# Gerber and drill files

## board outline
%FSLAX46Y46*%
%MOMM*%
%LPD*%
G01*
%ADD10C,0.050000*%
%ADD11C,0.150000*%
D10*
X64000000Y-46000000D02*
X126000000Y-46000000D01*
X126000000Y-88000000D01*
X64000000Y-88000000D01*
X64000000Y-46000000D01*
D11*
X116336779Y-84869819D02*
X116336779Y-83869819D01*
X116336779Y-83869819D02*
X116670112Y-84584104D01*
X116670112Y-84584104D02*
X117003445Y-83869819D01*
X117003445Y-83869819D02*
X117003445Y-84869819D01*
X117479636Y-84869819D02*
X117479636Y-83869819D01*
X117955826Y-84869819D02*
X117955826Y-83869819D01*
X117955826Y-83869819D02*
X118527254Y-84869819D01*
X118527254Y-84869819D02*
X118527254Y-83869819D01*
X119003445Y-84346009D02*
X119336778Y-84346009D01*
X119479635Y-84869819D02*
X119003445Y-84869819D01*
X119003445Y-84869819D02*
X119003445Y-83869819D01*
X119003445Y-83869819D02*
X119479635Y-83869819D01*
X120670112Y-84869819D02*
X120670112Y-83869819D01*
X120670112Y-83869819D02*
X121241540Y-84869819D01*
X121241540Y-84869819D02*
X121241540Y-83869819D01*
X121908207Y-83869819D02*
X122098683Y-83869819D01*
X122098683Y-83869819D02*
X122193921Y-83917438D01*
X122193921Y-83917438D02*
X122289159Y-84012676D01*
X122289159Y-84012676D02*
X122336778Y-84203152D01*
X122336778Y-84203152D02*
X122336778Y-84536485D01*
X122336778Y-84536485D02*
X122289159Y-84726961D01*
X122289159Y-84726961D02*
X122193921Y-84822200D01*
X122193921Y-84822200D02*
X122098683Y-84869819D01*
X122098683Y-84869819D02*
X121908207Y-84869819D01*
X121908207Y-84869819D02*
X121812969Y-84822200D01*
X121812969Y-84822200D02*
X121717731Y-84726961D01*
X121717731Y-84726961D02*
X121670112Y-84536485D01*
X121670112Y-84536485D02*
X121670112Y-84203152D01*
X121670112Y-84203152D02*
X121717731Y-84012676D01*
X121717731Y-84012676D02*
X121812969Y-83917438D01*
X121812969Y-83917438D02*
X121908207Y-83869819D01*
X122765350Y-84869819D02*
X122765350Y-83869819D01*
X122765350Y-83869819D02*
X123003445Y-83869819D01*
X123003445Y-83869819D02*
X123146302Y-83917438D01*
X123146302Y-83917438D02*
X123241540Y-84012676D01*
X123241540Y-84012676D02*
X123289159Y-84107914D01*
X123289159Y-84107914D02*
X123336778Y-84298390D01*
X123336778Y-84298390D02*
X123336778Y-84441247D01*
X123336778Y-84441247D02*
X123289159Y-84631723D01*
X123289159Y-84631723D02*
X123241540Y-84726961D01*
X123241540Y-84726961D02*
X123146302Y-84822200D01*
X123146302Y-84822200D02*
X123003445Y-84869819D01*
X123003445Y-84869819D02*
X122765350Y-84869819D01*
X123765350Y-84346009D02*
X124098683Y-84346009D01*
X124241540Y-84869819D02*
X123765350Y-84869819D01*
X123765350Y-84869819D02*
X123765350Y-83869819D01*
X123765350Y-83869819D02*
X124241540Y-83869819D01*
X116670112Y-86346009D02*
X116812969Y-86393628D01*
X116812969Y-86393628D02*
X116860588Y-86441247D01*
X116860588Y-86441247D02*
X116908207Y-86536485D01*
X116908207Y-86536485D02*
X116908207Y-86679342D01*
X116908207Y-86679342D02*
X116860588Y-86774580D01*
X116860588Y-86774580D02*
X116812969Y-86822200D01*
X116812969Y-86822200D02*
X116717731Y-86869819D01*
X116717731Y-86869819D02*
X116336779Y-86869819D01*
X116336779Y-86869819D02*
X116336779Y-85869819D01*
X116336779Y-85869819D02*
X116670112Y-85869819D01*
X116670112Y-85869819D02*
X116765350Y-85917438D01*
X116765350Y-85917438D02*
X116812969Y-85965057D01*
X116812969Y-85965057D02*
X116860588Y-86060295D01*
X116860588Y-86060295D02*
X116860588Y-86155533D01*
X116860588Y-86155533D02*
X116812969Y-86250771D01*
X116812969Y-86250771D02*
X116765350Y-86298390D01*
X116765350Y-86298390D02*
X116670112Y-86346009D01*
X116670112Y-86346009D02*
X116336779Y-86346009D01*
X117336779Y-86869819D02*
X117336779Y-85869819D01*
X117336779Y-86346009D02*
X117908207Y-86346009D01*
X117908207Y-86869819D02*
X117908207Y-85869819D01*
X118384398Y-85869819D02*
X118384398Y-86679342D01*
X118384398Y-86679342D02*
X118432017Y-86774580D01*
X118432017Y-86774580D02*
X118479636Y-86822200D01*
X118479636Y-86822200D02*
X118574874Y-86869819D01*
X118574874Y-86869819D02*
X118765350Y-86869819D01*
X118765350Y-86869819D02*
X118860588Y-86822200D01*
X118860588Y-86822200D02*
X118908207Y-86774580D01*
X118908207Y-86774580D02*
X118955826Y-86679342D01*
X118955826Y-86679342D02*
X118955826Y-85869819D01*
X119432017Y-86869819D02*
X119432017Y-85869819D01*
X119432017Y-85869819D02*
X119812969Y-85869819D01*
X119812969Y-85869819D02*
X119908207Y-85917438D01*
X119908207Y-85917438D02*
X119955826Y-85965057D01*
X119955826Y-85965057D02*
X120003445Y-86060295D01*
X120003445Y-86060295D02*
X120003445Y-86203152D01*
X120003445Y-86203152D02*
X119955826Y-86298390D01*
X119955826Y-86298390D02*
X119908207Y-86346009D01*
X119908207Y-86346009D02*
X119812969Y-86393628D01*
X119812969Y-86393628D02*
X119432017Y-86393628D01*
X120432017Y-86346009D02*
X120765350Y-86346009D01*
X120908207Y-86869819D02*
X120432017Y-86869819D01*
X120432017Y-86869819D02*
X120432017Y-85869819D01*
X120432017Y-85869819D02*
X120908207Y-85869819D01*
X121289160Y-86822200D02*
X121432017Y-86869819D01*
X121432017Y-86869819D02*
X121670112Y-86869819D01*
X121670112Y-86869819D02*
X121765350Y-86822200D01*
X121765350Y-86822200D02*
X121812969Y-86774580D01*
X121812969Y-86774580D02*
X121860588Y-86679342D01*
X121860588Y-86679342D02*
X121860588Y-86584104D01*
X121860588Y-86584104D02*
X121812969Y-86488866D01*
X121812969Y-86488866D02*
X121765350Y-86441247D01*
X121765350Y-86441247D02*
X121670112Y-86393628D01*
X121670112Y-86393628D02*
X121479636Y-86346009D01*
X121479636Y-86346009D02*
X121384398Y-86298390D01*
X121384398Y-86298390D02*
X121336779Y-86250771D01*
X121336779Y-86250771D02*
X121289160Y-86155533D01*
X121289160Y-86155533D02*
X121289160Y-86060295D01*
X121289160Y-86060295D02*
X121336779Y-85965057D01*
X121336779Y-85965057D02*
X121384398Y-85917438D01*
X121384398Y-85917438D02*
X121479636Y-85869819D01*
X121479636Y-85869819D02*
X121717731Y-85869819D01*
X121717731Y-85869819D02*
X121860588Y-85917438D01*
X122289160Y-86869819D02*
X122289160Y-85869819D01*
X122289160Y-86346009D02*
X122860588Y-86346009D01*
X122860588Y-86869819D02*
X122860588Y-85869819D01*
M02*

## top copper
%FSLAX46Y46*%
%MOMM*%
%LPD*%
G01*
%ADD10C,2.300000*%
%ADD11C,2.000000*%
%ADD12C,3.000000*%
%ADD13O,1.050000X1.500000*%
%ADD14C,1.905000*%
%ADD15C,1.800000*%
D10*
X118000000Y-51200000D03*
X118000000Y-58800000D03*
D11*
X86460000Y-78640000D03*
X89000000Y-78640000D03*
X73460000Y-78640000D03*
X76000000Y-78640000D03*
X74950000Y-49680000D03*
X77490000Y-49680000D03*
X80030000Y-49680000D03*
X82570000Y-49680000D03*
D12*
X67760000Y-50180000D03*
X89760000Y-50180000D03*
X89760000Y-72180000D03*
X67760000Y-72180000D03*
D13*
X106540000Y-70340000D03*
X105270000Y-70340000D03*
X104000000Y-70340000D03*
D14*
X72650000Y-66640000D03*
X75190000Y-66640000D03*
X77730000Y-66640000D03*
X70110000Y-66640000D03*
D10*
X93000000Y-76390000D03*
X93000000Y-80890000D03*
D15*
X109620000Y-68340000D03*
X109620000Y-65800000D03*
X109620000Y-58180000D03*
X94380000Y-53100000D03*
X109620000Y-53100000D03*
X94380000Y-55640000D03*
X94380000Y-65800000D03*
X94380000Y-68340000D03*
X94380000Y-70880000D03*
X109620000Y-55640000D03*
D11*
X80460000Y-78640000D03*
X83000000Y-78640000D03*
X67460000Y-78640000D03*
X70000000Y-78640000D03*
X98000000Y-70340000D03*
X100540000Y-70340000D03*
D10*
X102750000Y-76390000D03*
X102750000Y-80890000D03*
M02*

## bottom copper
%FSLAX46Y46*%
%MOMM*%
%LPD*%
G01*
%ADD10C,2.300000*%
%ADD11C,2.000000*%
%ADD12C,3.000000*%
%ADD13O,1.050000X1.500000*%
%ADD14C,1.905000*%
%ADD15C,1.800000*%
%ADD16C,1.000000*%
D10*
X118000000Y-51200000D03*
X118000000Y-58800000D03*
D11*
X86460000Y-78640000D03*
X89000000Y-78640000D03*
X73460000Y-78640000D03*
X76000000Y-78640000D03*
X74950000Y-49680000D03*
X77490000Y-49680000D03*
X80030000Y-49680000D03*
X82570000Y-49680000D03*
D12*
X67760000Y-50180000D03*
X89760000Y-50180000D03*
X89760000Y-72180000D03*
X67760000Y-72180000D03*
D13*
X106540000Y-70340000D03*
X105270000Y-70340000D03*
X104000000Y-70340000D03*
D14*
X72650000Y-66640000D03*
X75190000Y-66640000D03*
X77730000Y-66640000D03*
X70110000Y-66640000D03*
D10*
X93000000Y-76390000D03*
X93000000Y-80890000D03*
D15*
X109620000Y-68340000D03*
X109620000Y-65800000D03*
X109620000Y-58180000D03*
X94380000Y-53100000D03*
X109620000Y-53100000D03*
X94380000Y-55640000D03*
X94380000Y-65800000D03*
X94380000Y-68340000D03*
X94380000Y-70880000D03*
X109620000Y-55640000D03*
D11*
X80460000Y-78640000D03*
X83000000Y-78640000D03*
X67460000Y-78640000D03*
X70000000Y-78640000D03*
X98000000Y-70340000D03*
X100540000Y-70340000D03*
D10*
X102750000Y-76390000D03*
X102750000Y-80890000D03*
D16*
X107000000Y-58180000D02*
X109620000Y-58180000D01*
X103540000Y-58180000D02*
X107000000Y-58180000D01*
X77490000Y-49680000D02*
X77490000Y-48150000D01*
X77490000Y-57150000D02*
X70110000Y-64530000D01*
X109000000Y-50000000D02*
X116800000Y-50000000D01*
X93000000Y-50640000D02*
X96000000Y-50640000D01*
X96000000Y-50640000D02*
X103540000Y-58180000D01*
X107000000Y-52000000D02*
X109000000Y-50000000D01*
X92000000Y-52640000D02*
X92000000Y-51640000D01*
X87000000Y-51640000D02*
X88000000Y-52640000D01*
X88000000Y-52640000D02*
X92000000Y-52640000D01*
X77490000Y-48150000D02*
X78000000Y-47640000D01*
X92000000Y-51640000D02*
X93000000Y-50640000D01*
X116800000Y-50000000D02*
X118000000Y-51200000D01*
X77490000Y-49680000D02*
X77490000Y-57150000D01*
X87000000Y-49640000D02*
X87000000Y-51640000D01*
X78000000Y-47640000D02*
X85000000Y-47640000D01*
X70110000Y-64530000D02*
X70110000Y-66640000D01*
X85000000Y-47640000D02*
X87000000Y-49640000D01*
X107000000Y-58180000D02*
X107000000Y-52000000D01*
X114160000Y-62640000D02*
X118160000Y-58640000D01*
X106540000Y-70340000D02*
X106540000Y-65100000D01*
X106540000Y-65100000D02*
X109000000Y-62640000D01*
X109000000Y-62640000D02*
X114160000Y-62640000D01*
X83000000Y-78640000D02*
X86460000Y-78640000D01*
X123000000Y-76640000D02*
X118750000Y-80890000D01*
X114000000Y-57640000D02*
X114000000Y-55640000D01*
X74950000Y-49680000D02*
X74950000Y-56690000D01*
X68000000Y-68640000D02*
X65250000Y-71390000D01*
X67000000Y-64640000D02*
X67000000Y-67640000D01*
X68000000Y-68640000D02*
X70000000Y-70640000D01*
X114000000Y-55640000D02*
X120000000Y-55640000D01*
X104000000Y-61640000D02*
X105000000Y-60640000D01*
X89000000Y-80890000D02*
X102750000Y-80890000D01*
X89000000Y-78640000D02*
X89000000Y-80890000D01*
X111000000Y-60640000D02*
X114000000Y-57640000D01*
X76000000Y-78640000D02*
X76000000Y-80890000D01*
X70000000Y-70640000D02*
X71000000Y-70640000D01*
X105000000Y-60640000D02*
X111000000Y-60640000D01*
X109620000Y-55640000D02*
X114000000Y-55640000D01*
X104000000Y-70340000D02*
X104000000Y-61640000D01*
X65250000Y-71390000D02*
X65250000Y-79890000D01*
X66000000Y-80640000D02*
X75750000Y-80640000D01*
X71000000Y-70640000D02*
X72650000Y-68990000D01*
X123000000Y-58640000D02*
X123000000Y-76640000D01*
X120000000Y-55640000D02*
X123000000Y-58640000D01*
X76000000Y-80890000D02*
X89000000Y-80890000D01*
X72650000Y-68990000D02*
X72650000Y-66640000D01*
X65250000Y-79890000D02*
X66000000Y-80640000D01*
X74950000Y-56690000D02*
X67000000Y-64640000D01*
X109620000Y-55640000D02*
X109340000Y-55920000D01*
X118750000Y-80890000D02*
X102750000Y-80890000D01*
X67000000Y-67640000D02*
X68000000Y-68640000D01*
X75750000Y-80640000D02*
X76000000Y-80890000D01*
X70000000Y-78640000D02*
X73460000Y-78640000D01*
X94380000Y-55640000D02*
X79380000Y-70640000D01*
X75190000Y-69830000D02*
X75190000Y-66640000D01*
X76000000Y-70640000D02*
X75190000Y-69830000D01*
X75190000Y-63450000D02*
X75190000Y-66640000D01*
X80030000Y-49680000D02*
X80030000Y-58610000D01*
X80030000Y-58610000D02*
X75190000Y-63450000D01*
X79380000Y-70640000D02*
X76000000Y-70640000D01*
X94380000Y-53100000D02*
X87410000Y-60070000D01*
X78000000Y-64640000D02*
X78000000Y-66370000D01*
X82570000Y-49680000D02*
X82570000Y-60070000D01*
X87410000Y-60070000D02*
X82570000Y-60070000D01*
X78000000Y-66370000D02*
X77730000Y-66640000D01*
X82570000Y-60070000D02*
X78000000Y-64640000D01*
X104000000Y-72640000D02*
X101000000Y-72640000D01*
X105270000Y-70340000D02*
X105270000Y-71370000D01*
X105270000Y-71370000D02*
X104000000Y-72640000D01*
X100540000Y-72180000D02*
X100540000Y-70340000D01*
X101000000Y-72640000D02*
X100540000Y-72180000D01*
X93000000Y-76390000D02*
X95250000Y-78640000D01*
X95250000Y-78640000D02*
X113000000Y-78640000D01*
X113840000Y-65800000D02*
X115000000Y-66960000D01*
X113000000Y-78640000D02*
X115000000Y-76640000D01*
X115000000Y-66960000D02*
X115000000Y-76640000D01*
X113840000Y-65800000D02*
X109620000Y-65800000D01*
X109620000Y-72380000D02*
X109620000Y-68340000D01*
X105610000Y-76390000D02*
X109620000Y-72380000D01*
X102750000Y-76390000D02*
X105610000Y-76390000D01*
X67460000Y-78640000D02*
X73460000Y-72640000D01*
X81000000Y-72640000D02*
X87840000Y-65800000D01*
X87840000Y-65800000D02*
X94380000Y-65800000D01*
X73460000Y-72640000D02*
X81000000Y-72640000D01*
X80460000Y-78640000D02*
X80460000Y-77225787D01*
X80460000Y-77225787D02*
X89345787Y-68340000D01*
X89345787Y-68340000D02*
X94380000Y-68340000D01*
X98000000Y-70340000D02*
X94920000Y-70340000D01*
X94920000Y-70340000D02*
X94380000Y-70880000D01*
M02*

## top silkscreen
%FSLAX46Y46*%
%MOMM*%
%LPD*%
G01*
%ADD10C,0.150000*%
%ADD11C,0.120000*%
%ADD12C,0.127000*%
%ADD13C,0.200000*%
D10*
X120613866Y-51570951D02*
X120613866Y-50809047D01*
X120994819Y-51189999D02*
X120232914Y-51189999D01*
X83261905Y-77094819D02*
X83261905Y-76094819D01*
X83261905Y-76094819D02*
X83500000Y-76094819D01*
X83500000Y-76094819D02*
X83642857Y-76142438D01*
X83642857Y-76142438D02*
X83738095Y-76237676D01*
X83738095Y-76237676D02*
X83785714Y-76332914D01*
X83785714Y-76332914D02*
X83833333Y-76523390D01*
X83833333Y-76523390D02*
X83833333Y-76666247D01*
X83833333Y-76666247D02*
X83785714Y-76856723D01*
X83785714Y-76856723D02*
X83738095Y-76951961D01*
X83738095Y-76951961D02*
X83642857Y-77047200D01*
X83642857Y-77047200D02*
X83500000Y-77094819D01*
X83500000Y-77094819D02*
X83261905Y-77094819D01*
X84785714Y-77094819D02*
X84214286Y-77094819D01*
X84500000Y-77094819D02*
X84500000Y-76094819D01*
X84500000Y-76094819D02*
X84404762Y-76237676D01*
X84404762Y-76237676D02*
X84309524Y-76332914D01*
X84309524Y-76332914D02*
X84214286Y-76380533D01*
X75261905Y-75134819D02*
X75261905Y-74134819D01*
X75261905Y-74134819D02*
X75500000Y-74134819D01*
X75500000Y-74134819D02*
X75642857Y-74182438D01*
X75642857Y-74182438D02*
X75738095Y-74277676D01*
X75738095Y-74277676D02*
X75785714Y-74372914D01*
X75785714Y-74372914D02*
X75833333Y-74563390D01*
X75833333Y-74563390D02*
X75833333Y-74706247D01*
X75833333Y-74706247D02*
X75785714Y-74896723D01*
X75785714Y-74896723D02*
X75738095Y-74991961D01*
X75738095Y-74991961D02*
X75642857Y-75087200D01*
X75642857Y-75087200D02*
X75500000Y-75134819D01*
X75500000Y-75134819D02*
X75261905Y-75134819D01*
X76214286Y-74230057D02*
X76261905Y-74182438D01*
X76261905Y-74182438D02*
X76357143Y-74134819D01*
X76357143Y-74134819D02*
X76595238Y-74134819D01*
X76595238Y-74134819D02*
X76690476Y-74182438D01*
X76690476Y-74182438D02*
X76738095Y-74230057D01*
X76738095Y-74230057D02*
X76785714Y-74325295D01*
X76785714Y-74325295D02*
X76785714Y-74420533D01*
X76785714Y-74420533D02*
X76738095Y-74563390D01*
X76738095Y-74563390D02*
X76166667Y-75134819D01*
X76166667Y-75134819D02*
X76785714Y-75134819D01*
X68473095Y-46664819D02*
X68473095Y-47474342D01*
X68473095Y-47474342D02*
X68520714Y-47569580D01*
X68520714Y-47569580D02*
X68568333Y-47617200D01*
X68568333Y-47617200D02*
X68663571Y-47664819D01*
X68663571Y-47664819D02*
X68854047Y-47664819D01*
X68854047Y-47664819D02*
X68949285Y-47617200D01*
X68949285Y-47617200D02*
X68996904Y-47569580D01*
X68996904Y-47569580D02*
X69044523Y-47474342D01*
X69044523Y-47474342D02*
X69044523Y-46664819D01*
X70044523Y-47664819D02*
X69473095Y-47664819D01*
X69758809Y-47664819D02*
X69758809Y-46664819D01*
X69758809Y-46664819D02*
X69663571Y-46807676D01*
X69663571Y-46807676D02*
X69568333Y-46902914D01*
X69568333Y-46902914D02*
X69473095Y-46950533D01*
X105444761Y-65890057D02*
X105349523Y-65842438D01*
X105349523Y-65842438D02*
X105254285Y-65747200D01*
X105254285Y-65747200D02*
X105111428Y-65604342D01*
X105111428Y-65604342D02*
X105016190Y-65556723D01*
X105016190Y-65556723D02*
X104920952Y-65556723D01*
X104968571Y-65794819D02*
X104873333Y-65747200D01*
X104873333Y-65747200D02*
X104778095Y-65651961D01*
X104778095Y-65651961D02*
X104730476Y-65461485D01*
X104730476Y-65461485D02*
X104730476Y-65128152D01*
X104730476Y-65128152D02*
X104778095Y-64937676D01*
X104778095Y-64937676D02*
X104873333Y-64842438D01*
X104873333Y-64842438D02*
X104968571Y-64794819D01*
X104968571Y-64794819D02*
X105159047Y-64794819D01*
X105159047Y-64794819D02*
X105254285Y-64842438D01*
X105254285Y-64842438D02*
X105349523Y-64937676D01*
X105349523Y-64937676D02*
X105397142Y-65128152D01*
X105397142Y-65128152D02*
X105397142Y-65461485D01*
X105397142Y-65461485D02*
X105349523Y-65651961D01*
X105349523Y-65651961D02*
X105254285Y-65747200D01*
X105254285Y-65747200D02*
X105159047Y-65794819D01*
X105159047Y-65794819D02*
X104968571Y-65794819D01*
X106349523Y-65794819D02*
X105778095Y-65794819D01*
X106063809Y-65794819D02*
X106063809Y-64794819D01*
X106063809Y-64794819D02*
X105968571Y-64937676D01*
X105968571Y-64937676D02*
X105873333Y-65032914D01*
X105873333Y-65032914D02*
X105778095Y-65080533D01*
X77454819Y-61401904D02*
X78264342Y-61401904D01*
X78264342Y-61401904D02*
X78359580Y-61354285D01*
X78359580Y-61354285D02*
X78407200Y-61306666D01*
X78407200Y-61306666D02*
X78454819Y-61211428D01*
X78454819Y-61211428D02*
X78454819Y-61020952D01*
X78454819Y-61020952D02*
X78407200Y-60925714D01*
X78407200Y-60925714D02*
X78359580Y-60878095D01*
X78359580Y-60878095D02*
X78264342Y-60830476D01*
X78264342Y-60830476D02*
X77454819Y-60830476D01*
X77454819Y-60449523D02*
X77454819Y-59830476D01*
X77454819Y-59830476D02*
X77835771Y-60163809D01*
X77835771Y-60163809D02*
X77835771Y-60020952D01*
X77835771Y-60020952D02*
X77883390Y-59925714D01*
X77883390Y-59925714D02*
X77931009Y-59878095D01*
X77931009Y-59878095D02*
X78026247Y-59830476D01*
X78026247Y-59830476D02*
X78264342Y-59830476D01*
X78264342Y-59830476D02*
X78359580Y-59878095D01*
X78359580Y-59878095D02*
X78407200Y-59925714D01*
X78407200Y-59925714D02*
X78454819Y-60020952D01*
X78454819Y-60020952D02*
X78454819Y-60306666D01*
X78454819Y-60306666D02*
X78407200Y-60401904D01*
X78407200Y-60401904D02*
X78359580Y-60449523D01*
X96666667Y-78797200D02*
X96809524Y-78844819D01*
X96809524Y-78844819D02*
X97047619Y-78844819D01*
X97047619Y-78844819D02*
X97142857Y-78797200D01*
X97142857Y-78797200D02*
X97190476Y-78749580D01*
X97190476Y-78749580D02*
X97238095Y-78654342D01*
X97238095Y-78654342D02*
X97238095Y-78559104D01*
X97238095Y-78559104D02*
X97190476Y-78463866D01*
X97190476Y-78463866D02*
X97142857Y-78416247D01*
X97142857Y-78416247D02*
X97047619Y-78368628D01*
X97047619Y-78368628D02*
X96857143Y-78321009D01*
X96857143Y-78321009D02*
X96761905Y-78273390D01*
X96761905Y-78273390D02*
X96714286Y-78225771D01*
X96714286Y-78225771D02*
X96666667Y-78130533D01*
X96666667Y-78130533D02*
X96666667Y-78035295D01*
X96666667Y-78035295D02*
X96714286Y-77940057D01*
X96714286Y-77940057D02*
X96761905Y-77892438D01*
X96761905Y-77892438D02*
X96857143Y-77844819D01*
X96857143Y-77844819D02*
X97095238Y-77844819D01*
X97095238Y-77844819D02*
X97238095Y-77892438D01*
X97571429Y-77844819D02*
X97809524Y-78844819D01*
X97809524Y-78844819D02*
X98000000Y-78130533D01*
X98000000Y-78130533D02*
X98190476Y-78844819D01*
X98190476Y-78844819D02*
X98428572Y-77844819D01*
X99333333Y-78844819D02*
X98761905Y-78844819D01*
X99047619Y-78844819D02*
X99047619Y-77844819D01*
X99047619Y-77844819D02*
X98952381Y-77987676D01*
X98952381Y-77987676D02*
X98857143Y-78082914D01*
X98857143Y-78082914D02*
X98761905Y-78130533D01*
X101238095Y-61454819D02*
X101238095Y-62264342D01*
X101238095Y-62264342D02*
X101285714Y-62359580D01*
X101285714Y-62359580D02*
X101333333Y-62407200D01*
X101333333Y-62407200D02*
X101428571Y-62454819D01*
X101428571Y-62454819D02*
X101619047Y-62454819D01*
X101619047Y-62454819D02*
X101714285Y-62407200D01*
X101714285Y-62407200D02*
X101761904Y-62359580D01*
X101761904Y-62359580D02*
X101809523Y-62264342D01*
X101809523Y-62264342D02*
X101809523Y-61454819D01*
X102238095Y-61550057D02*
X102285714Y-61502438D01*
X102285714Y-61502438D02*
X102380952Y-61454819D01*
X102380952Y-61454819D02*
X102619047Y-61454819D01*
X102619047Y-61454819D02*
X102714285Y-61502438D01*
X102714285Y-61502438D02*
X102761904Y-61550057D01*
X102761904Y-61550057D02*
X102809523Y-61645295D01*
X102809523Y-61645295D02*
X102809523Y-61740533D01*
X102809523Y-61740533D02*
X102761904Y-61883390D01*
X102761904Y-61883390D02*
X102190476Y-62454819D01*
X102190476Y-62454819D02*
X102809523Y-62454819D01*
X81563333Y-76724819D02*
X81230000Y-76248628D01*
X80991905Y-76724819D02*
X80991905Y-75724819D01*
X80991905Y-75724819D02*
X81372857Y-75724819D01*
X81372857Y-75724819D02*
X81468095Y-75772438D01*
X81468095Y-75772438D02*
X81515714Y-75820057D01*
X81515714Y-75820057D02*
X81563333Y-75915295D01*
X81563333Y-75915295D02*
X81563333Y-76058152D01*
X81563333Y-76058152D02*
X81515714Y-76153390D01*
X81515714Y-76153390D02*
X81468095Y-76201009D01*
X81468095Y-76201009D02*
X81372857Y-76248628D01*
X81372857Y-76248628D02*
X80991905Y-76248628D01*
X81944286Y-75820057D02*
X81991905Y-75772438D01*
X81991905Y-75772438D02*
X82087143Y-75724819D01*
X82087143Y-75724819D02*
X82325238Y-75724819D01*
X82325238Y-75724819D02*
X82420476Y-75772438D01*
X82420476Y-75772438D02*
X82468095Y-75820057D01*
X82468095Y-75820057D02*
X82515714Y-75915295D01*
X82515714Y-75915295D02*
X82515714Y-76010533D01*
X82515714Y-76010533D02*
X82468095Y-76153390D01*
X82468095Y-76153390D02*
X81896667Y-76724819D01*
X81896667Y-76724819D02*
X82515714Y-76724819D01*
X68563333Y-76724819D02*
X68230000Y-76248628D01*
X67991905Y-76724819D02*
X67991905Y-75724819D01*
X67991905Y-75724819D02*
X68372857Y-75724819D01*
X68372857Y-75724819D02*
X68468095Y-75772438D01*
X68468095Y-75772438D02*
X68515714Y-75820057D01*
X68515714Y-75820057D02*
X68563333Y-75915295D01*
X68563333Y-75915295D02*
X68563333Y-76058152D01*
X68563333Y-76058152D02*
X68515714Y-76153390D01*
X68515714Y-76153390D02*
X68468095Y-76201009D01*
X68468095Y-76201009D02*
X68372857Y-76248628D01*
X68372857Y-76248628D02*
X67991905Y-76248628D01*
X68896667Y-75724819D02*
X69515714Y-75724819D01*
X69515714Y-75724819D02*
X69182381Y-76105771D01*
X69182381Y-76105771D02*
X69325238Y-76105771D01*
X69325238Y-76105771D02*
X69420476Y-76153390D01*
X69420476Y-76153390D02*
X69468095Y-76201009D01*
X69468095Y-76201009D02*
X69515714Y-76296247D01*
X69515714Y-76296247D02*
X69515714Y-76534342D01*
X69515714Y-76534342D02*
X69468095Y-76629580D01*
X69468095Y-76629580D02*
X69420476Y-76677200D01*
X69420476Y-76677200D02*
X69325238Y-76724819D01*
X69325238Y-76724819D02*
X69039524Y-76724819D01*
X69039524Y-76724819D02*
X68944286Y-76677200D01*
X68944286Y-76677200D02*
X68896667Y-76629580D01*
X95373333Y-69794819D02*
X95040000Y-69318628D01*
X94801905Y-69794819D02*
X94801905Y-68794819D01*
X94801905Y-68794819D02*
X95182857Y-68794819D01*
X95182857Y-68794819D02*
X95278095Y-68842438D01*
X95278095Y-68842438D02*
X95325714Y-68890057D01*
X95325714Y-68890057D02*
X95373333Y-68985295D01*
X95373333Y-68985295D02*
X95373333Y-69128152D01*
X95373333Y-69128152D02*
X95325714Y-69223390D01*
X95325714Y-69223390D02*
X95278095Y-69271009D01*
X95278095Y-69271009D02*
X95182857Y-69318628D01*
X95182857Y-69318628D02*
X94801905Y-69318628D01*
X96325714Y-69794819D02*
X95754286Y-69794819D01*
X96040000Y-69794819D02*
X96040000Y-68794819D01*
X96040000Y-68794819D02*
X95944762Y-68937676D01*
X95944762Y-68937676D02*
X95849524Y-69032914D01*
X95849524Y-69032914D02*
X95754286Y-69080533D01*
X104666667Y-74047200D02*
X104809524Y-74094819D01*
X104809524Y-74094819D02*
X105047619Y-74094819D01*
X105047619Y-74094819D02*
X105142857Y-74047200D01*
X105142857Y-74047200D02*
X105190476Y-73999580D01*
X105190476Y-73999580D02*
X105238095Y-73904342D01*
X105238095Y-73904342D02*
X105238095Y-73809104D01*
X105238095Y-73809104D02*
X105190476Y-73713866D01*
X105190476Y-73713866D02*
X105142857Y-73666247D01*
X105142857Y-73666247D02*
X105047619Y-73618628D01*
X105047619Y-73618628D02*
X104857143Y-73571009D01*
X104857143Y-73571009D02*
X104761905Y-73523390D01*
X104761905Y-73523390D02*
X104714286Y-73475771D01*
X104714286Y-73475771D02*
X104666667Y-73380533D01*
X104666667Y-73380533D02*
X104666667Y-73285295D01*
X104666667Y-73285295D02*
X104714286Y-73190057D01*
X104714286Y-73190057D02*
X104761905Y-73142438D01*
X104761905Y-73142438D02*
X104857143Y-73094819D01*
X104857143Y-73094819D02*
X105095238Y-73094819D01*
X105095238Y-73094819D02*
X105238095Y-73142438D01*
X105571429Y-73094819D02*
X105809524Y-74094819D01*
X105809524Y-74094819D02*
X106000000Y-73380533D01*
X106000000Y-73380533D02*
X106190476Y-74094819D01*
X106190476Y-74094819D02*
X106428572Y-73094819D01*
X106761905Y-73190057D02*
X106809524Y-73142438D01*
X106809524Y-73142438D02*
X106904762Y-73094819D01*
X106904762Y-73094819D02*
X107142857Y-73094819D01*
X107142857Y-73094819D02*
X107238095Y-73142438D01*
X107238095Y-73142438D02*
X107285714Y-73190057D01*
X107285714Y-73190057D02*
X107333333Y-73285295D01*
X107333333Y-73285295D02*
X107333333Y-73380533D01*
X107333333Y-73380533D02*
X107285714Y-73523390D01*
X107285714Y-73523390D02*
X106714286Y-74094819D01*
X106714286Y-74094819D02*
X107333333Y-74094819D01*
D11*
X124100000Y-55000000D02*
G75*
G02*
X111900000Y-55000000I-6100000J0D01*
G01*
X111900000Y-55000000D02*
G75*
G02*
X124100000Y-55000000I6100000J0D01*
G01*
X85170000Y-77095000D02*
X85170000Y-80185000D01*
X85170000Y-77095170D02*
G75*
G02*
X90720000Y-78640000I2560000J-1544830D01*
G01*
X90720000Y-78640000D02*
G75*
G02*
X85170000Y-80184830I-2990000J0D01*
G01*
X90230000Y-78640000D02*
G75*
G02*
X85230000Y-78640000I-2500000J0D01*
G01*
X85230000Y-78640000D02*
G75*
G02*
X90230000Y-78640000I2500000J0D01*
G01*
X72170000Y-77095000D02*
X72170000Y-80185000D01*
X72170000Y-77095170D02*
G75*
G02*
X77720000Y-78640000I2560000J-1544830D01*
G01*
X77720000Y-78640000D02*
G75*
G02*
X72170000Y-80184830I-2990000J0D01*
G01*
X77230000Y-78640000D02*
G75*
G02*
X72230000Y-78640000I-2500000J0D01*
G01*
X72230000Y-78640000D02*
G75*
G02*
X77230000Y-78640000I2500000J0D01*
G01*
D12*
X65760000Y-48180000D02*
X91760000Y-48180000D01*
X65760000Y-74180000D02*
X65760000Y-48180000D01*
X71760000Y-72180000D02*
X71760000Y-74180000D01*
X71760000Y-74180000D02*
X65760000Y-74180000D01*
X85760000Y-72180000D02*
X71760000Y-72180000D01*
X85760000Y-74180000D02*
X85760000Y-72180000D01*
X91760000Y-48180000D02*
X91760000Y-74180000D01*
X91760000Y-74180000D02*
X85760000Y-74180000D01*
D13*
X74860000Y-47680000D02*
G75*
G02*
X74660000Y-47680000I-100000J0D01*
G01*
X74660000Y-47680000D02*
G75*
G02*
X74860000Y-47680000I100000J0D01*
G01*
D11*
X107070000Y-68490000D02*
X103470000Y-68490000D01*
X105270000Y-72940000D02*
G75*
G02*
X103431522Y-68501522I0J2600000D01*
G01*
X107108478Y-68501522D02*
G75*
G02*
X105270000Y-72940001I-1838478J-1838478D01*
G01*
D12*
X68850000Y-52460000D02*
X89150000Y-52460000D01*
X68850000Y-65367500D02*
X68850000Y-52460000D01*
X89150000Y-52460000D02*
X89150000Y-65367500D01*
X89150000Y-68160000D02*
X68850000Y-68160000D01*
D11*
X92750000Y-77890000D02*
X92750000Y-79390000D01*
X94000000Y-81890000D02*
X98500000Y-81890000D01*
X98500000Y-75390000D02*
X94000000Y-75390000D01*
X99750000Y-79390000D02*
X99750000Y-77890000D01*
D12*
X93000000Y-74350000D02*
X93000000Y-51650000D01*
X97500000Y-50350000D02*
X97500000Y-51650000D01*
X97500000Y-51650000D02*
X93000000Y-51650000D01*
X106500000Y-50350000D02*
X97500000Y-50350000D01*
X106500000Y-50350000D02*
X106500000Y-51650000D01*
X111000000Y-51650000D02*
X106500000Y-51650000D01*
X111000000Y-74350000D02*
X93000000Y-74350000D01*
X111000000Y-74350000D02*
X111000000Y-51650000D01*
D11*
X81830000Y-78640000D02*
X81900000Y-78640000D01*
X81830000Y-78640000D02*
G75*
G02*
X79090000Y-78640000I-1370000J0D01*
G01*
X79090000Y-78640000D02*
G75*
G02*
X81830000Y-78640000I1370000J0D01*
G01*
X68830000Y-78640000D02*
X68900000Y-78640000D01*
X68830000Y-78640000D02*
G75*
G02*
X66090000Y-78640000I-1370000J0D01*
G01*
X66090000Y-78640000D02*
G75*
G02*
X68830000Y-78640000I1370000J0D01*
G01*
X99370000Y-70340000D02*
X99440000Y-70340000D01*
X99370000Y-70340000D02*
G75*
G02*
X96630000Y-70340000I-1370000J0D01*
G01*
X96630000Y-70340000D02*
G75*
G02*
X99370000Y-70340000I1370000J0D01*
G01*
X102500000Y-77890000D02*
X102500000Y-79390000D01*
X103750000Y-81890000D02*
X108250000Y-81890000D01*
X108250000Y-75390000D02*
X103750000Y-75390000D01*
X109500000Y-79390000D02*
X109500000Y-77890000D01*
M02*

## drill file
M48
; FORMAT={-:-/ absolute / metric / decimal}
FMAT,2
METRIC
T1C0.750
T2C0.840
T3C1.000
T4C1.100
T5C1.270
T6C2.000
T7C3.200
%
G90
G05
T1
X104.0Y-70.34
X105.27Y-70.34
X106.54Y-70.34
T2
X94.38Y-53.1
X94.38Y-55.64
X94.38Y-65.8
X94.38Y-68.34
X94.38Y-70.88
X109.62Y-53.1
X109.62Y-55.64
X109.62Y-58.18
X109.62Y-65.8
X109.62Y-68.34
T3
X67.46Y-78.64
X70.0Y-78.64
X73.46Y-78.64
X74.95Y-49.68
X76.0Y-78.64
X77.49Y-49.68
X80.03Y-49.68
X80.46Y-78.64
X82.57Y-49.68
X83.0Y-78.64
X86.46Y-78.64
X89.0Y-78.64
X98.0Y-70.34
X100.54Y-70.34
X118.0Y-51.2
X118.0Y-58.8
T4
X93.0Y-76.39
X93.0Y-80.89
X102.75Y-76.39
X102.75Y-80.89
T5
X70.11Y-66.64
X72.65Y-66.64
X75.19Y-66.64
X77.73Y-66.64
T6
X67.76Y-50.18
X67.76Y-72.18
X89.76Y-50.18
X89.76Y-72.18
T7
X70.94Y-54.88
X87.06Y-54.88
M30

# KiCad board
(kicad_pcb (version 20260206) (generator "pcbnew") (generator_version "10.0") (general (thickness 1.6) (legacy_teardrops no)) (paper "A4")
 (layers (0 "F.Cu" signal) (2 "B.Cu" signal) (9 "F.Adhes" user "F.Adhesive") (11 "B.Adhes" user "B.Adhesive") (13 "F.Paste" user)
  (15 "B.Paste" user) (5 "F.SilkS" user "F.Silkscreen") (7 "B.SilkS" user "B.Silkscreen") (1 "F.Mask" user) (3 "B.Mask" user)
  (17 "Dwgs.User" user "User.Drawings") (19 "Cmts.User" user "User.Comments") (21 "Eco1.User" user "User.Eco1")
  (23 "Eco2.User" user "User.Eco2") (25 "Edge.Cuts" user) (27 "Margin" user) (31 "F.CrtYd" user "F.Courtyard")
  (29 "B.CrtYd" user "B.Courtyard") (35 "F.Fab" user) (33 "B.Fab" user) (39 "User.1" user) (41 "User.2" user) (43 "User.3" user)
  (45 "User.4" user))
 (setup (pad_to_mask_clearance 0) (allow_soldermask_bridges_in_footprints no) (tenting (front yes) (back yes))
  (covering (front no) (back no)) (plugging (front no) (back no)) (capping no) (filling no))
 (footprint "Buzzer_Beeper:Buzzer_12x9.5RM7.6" (layer "F.Cu") (at 118 51.2 -90)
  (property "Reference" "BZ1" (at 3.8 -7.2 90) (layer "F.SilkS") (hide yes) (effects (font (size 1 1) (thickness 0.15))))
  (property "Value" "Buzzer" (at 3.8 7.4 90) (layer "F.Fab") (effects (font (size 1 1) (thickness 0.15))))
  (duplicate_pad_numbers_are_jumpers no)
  (fp_circle (center 3.8 0) (end 9.9 0) (stroke (width 0.12) (type solid)) (fill no) (layer "F.SilkS"))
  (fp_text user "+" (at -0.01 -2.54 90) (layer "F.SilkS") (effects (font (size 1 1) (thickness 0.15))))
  (pad "1" thru_hole circle (at 0 0 270) (size 2.3 2.3) (drill 1) (layers "*.Cu" "*.Mask") (remove_unused_layers no) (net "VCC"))
  (pad "2" thru_hole circle (at 7.6 0 270) (size 2.3 2.3) (drill 1) (layers "*.Cu" "*.Mask") (remove_unused_layers no) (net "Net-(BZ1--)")))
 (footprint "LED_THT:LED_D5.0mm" (layer "F.Cu") (at 86.46 78.64)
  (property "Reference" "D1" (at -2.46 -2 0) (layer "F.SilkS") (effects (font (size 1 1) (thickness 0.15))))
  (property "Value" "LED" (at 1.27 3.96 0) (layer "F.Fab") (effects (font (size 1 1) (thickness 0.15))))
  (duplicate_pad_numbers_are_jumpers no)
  (fp_line (start -1.29 -1.545) (end -1.29 1.545) (stroke (width 0.12) (type solid)) (layer "F.SilkS"))
  (fp_arc (start -1.29 -1.54483) (mid 2.071779 -2.880495) (end 4.26 0) (stroke (width 0.12) (type solid)) (layer "F.SilkS"))
  (fp_arc (start 4.26 0) (mid 2.071779 2.880495) (end -1.29 1.54483) (stroke (width 0.12) (type solid)) (layer "F.SilkS"))
  (fp_circle (center 1.27 0) (end 3.77 0) (stroke (width 0.12) (type solid)) (fill no) (layer "F.SilkS"))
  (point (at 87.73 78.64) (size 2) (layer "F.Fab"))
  (pad "1" thru_hole circle (at 0 0) (size 2 2) (drill 1) (layers "*.Cu" "*.Mask") (remove_unused_layers no) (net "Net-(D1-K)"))
  (pad "2" thru_hole circle (at 2.54 0) (size 2 2) (drill 1) (layers "*.Cu" "*.Mask") (remove_unused_layers no) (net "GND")))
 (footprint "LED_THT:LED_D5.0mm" (layer "F.Cu") (at 73.46 78.64)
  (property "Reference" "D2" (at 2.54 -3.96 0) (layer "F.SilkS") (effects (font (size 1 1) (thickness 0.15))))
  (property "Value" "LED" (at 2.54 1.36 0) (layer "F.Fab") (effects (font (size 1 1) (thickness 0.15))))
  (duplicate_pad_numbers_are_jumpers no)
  (fp_line (start -1.29 -1.545) (end -1.29 1.545) (stroke (width 0.12) (type solid)) (layer "F.SilkS"))
  (fp_arc (start -1.29 -1.54483) (mid 2.071779 -2.880495) (end 4.26 0) (stroke (width 0.12) (type solid)) (layer "F.SilkS"))
  (fp_arc (start 4.26 0) (mid 2.071779 2.880495) (end -1.29 1.54483) (stroke (width 0.12) (type solid)) (layer "F.SilkS"))
  (fp_circle (center 1.27 0) (end 3.77 0) (stroke (width 0.12) (type solid)) (fill no) (layer "F.SilkS"))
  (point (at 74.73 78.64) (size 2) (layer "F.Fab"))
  (pad "1" thru_hole circle (at 0 0) (size 2 2) (drill 1) (layers "*.Cu" "*.Mask") (remove_unused_layers no) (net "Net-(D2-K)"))
  (pad "2" thru_hole circle (at 2.54 0) (size 2 2) (drill 1) (layers "*.Cu" "*.Mask") (remove_unused_layers no) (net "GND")))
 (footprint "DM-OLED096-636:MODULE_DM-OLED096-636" (layer "F.Cu") (at 78.76 61.18)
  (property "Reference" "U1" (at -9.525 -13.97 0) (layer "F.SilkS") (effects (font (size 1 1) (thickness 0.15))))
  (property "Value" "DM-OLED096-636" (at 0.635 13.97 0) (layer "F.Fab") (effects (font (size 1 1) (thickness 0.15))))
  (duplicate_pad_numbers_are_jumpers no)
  (fp_line (start -13 -13) (end 13 -13) (stroke (width 0.127) (type solid)) (layer "F.SilkS"))
  (fp_line (start -13 13) (end -13 -13) (stroke (width 0.127) (type solid)) (layer "F.SilkS"))
  (fp_line (start -7 11) (end -7 13) (stroke (width 0.127) (type solid)) (layer "F.SilkS"))
  (fp_line (start -7 13) (end -13 13) (stroke (width 0.127) (type solid)) (layer "F.SilkS"))
  (fp_line (start 7 11) (end -7 11) (stroke (width 0.127) (type solid)) (layer "F.SilkS"))
  (fp_line (start 7 13) (end 7 11) (stroke (width 0.127) (type solid)) (layer "F.SilkS"))
  (fp_line (start 13 -13) (end 13 13) (stroke (width 0.127) (type solid)) (layer "F.SilkS"))
  (fp_line (start 13 13) (end 7 13) (stroke (width 0.127) (type solid)) (layer "F.SilkS"))
  (fp_circle (center -4 -13.5) (end -3.9 -13.5) (stroke (width 0.2) (type solid)) (fill no) (layer "F.SilkS"))
  (pad "1" thru_hole circle (at -3.81 -11.5) (size 2 2) (drill 1) (layers "*.Cu" "*.Mask") (remove_unused_layers no) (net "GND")
   (solder_mask_margin 0.102))
  (pad "2" thru_hole circle (at -1.27 -11.5) (size 2 2) (drill 1) (layers "*.Cu" "*.Mask") (remove_unused_layers no) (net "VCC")
   (solder_mask_margin 0.102))
  (pad "3" thru_hole circle (at 1.27 -11.5) (size 2 2) (drill 1) (layers "*.Cu" "*.Mask") (remove_unused_layers no) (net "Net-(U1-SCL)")
   (solder_mask_margin 0.102))
  (pad "4" thru_hole circle (at 3.81 -11.5) (size 2 2) (drill 1) (layers "*.Cu" "*.Mask") (remove_unused_layers no) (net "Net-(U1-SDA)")
   (solder_mask_margin 0.102))
  (pad "S1" thru_hole circle (at -11 -11) (size 3 3) (drill 2) (layers "*.Cu" "*.Mask") (remove_unused_layers no) (solder_mask_margin 0.102))
  (pad "S2" thru_hole circle (at 11 -11) (size 3 3) (drill 2) (layers "*.Cu" "*.Mask") (remove_unused_layers no) (solder_mask_margin 0.102))
  (pad "S3" thru_hole circle (at 11 11) (size 3 3) (drill 2) (layers "*.Cu" "*.Mask") (remove_unused_layers no) (solder_mask_margin 0.102))
  (pad "S4" thru_hole circle (at -11 11) (size 3 3) (drill 2) (layers "*.Cu" "*.Mask") (remove_unused_layers no) (solder_mask_margin 0.102)))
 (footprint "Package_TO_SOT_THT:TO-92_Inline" (layer "F.Cu") (at 106.54 70.34 180)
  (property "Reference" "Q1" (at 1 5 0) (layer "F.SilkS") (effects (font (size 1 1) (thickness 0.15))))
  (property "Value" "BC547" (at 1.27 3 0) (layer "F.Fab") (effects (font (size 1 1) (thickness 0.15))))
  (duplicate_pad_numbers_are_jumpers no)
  (fp_line (start -0.53 1.85) (end 3.07 1.85) (stroke (width 0.12) (type solid)) (layer "F.SilkS"))
  (fp_arc (start 1.27 -2.6) (mid 3.672087 -0.994977) (end 3.108478 1.838478) (stroke (width 0.12) (type solid)) (layer "F.SilkS"))
  (fp_arc (start -0.568478 1.838478) (mid -1.132087 -0.994977) (end 1.27 -2.6) (stroke (width 0.12) (type solid)) (layer "F.SilkS"))
  (pad "1" thru_hole oval (at 0 0 180) (size 1.05 1.5) (drill 0.75) (layers "*.Cu" "*.Mask") (remove_unused_layers no) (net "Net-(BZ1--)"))
  (pad "2" thru_hole oval (at 1.27 0 180) (size 1.05 1.5) (drill 0.75) (layers "*.Cu" "*.Mask") (remove_unused_layers no) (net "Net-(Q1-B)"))
  (pad "3" thru_hole oval (at 2.54 0 180) (size 1.05 1.5) (drill 0.75) (layers "*.Cu" "*.Mask") (remove_unused_layers no) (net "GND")))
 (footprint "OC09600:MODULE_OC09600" (layer "F.Cu") (at 79 60.31 90)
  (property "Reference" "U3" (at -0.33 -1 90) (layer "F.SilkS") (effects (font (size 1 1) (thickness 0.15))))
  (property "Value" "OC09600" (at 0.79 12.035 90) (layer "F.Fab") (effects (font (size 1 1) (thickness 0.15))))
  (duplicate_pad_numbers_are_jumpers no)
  (fp_line (start 7.85 -10.15) (end 7.85 10.15) (stroke (width 0.127) (type solid)) (layer "F.SilkS"))
  (fp_line (start -5.0575 -10.15) (end 7.85 -10.15) (stroke (width 0.127) (type solid)) (layer "F.SilkS"))
  (fp_line (start 7.85 10.15) (end -5.0575 10.15) (stroke (width 0.127) (type solid)) (layer "F.SilkS"))
  (fp_line (start -7.85 10.15) (end -7.85 -10.15) (stroke (width 0.127) (type solid)) (layer "F.SilkS"))
  (pad "" np_thru_hole circle (at 5.43 -8.06 90) (size 3.2 3.2) (drill 3.2) (layers "*.Cu" "*.Mask"))
  (pad "" np_thru_hole circle (at 5.43 8.06 90) (size 3.2 3.2) (drill 3.2) (layers "*.Cu" "*.Mask"))
  (pad "GND" thru_hole circle (at -6.33 -6.35 90) (size 1.905 1.905) (drill 1.27) (layers "*.Cu" "*.Mask") (remove_unused_layers no)
   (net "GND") (solder_mask_margin 0.102))
  (pad "SCL" thru_hole circle (at -6.33 -3.81 90) (size 1.905 1.905) (drill 1.27) (layers "*.Cu" "*.Mask") (remove_unused_layers no)
   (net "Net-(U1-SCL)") (solder_mask_margin 0.102))
  (pad "SDA" thru_hole circle (at -6.33 -1.27 90) (size 1.905 1.905) (drill 1.27) (layers "*.Cu" "*.Mask") (remove_unused_layers no)
   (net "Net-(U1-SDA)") (solder_mask_margin 0.102))
  (pad "VCC" thru_hole circle (at -6.33 -8.89 90) (size 1.905 1.905) (drill 1.27) (layers "*.Cu" "*.Mask") (remove_unused_layers no)
   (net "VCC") (solder_mask_margin 0.102)))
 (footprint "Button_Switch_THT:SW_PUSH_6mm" (layer "F.Cu") (at 93 76.39)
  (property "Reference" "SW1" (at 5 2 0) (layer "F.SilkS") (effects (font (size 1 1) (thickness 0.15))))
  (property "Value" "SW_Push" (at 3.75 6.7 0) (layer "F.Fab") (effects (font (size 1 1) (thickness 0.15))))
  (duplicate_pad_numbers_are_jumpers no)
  (fp_line (start -0.25 1.5) (end -0.25 3) (stroke (width 0.12) (type solid)) (layer "F.SilkS"))
  (fp_line (start 1 5.5) (end 5.5 5.5) (stroke (width 0.12) (type solid)) (layer "F.SilkS"))
  (fp_line (start 5.5 -1) (end 1 -1) (stroke (width 0.12) (type solid)) (layer "F.SilkS"))
  (fp_line (start 6.75 3) (end 6.75 1.5) (stroke (width 0.12) (type solid)) (layer "F.SilkS"))
  (pad "1" thru_hole circle (at 0 0 90) (size 2.3 2.3) (drill 1.1) (layers "*.Cu" "*.Mask") (remove_unused_layers no) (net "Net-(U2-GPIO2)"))
  (pad "2" thru_hole circle (at 0 4.5 90) (size 2.3 2.3) (drill 1.1) (layers "*.Cu" "*.Mask") (remove_unused_layers no) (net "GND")))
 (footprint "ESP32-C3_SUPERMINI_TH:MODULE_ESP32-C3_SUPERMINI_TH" (layer "F.Cu") (at 102 63)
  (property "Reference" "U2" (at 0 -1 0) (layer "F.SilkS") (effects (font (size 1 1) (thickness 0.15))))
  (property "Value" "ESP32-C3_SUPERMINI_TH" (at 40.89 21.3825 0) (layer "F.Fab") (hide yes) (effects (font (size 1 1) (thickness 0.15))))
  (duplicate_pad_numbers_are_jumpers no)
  (fp_line (start -9 11.35) (end -9 -11.35) (stroke (width 0.127) (type solid)) (layer "F.SilkS"))
  (fp_line (start -4.5 -12.65) (end -4.5 -11.35) (stroke (width 0.127) (type solid)) (layer "F.SilkS"))
  (fp_line (start -4.5 -11.35) (end -9 -11.35) (stroke (width 0.127) (type solid)) (layer "F.SilkS"))
  (fp_line (start 4.5 -12.65) (end -4.5 -12.65) (stroke (width 0.127) (type solid)) (layer "F.SilkS"))
  (fp_line (start 4.5 -12.65) (end 4.5 -11.35) (stroke (width 0.127) (type solid)) (layer "F.SilkS"))
  (fp_line (start 9 -11.35) (end 4.5 -11.35) (stroke (width 0.127) (type solid)) (layer "F.SilkS"))
  (fp_line (start 9 11.35) (end -9 11.35) (stroke (width 0.127) (type solid)) (layer "F.SilkS"))
  (fp_line (start 9 11.35) (end 9 -11.35) (stroke (width 0.127) (type solid)) (layer "F.SilkS"))
  (pad "1" thru_hole circle (at 7.62 5.34) (size 1.8 1.8) (drill 0.84) (layers "*.Cu" "*.Mask") (remove_unused_layers no)
   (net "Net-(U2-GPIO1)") (solder_mask_margin 0.102))
  (pad "2" thru_hole circle (at 7.62 2.8) (size 1.8 1.8) (drill 0.84) (layers "*.Cu" "*.Mask") (remove_unused_layers no)
   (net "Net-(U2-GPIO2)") (solder_mask_margin 0.102))
  (pad "3.3" thru_hole circle (at 7.62 -4.82) (size 1.8 1.8) (drill 0.84) (layers "*.Cu" "*.Mask") (remove_unused_layers no) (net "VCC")
   (solder_mask_margin 0.102))
  (pad "5" thru_hole circle (at -7.62 -9.9) (size 1.8 1.8) (drill 0.84) (layers "*.Cu" "*.Mask") (remove_unused_layers no)
   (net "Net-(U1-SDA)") (solder_mask_margin 0.102))
  (pad "5V" thru_hole circle (at 7.62 -9.9) (size 1.8 1.8) (drill 0.84) (layers "*.Cu" "*.Mask") (remove_unused_layers no)
   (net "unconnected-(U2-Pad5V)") (solder_mask_margin 0.102))
  (pad "6" thru_hole circle (at -7.62 -7.36) (size 1.8 1.8) (drill 0.84) (layers "*.Cu" "*.Mask") (remove_unused_layers no)
   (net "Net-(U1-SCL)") (solder_mask_margin 0.102))
  (pad "10" thru_hole circle (at -7.62 2.8) (size 1.8 1.8) (drill 0.84) (layers "*.Cu" "*.Mask") (remove_unused_layers no)
   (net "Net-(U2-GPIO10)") (solder_mask_margin 0.102))
  (pad "20" thru_hole circle (at -7.62 5.34) (size 1.8 1.8) (drill 0.84) (layers "*.Cu" "*.Mask") (remove_unused_layers no)
   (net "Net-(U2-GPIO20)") (solder_mask_margin 0.102))
  (pad "21" thru_hole circle (at -7.62 7.88) (size 1.8 1.8) (drill 0.84) (layers "*.Cu" "*.Mask") (remove_unused_layers no)
   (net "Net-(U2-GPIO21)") (solder_mask_margin 0.102))
  (pad "G" thru_hole circle (at 7.62 -7.36) (size 1.8 1.8) (drill 0.84) (layers "*.Cu" "*.Mask") (remove_unused_layers no) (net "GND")
   (solder_mask_margin 0.102)))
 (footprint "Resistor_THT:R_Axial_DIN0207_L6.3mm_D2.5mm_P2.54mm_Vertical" (layer "F.Cu") (at 80.46 78.64)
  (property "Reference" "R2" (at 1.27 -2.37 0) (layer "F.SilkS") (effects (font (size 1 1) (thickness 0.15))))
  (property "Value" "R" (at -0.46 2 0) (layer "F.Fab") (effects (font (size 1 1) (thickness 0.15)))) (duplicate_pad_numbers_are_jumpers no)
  (fp_line (start 1.37 0) (end 1.44 0) (stroke (width 0.12) (type solid)) (layer "F.SilkS"))
  (fp_circle (center 0 0) (end 1.37 0) (stroke (width 0.12) (type solid)) (fill no) (layer "F.SilkS"))
  (pad "1" thru_hole circle (at 0 0) (size 2 2) (drill 1) (layers "*.Cu" "*.Mask") (remove_unused_layers no) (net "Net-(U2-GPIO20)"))
  (pad "2" thru_hole circle (at 2.54 0) (size 2 2) (drill 1) (layers "*.Cu" "*.Mask") (remove_unused_layers no) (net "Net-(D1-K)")))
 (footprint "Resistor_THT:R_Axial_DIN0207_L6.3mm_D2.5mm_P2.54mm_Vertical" (layer "F.Cu") (at 67.46 78.64)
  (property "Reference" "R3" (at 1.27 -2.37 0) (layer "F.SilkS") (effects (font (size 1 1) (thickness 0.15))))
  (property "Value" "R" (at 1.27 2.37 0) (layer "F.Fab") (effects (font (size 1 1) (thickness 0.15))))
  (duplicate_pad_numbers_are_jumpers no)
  (fp_line (start 1.37 0) (end 1.44 0) (stroke (width 0.12) (type solid)) (layer "F.SilkS"))
  (fp_circle (center 0 0) (end 1.37 0) (stroke (width 0.12) (type solid)) (fill no) (layer "F.SilkS"))
  (pad "1" thru_hole circle (at 0 0) (size 2 2) (drill 1) (layers "*.Cu" "*.Mask") (remove_unused_layers no) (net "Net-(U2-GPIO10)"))
  (pad "2" thru_hole circle (at 2.54 0) (size 2 2) (drill 1) (layers "*.Cu" "*.Mask") (remove_unused_layers no) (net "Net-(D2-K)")))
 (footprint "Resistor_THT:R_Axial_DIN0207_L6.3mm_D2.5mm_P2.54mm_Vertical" (layer "F.Cu") (at 98 70.34)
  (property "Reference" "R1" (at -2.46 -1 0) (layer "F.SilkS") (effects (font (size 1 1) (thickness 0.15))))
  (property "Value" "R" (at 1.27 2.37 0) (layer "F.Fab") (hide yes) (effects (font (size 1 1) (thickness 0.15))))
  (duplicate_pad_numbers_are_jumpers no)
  (fp_line (start 1.37 0) (end 1.44 0) (stroke (width 0.12) (type solid)) (layer "F.SilkS"))
  (fp_circle (center 0 0) (end 1.37 0) (stroke (width 0.12) (type solid)) (fill no) (layer "F.SilkS"))
  (pad "1" thru_hole circle (at 0 0) (size 2 2) (drill 1) (layers "*.Cu" "*.Mask") (remove_unused_layers no) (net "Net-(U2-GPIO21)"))
  (pad "2" thru_hole circle (at 2.54 0) (size 2 2) (drill 1) (layers "*.Cu" "*.Mask") (remove_unused_layers no) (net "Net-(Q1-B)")))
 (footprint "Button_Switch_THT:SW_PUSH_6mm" (layer "F.Cu") (at 102.75 76.39)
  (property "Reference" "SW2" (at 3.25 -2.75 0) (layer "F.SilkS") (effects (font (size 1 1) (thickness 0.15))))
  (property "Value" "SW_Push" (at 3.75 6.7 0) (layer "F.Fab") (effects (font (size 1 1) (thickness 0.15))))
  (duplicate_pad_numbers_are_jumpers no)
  (fp_line (start -0.25 1.5) (end -0.25 3) (stroke (width 0.12) (type solid)) (layer "F.SilkS"))
  (fp_line (start 1 5.5) (end 5.5 5.5) (stroke (width 0.12) (type solid)) (layer "F.SilkS"))
  (fp_line (start 5.5 -1) (end 1 -1) (stroke (width 0.12) (type solid)) (layer "F.SilkS"))
  (fp_line (start 6.75 3) (end 6.75 1.5) (stroke (width 0.12) (type solid)) (layer "F.SilkS"))
  (pad "1" thru_hole circle (at 0 0 90) (size 2.3 2.3) (drill 1.1) (layers "*.Cu" "*.Mask") (remove_unused_layers no) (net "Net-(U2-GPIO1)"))
  (pad "2" thru_hole circle (at 0 4.5 90) (size 2.3 2.3) (drill 1.1) (layers "*.Cu" "*.Mask") (remove_unused_layers no) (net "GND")))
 (gr_rect (start 64 46) (end 126 88) (stroke (width 0.05) (type default)) (fill no) (layer "Edge.Cuts"))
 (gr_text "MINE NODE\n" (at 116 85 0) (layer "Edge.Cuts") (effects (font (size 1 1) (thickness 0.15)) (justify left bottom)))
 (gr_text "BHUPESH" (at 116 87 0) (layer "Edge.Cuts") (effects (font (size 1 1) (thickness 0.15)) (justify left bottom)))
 (segment (start 107 58.18) (end 109.62 58.18) (width 1) (layer "B.Cu") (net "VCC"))
 (segment (start 103.54 58.18) (end 107 58.18) (width 1) (layer "B.Cu") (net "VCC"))
 (segment (start 77.49 49.68) (end 77.49 48.15) (width 1) (layer "B.Cu") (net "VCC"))
 (segment (start 77.49 57.15) (end 70.11 64.53) (width 1) (layer "B.Cu") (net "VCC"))
 (segment (start 109 50) (end 116.8 50) (width 1) (layer "B.Cu") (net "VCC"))
 (segment (start 93 50.64) (end 96 50.64) (width 1) (layer "B.Cu") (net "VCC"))
 (segment (start 96 50.64) (end 103.54 58.18) (width 1) (layer "B.Cu") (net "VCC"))
 (segment (start 107 52) (end 109 50) (width 1) (layer "B.Cu") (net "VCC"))
 (segment (start 92 52.64) (end 92 51.64) (width 1) (layer "B.Cu") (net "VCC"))
 (segment (start 87 51.64) (end 88 52.64) (width 1) (layer "B.Cu") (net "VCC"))
 (segment (start 88 52.64) (end 92 52.64) (width 1) (layer "B.Cu") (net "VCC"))
 (segment (start 77.49 48.15) (end 78 47.64) (width 1) (layer "B.Cu") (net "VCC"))
 (segment (start 92 51.64) (end 93 50.64) (width 1) (layer "B.Cu") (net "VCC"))
 (segment (start 116.8 50) (end 118 51.2) (width 1) (layer "B.Cu") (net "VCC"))
 (segment (start 77.49 49.68) (end 77.49 57.15) (width 1) (layer "B.Cu") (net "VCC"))
 (segment (start 87 49.64) (end 87 51.64) (width 1) (layer "B.Cu") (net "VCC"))
 (segment (start 78 47.64) (end 85 47.64) (width 1) (layer "B.Cu") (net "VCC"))
 (segment (start 70.11 64.53) (end 70.11 66.64) (width 1) (layer "B.Cu") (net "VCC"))
 (segment (start 85 47.64) (end 87 49.64) (width 1) (layer "B.Cu") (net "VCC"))
 (segment (start 107 58.18) (end 107 52) (width 1) (layer "B.Cu") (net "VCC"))
 (segment (start 114.16 62.64) (end 118.16 58.64) (width 1) (layer "B.Cu") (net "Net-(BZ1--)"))
 (segment (start 106.54 70.34) (end 106.54 65.1) (width 1) (layer "B.Cu") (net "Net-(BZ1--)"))
 (segment (start 106.54 65.1) (end 109 62.64) (width 1) (layer "B.Cu") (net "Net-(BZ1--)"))
 (segment (start 109 62.64) (end 114.16 62.64) (width 1) (layer "B.Cu") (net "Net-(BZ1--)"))
 (segment (start 83 78.64) (end 86.46 78.64) (width 1) (layer "B.Cu") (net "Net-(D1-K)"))
 (segment (start 123 76.64) (end 118.75 80.89) (width 1) (layer "B.Cu") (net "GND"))
 (segment (start 114 57.64) (end 114 55.64) (width 1) (layer "B.Cu") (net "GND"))
 (segment (start 74.95 49.68) (end 74.95 56.69) (width 1) (layer "B.Cu") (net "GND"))
 (segment (start 68 68.64) (end 65.25 71.39) (width 1) (layer "B.Cu") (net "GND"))
 (segment (start 67 64.64) (end 67 67.64) (width 1) (layer "B.Cu") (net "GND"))
 (segment (start 68 68.64) (end 70 70.64) (width 1) (layer "B.Cu") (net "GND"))
 (segment (start 114 55.64) (end 120 55.64) (width 1) (layer "B.Cu") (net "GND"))
 (segment (start 104 61.64) (end 105 60.64) (width 1) (layer "B.Cu") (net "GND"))
 (segment (start 89 80.89) (end 102.75 80.89) (width 1) (layer "B.Cu") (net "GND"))
 (segment (start 89 78.64) (end 89 80.89) (width 1) (layer "B.Cu") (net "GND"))
 (segment (start 111 60.64) (end 114 57.64) (width 1) (layer "B.Cu") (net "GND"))
 (segment (start 76 78.64) (end 76 80.89) (width 1) (layer "B.Cu") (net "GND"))
 (segment (start 70 70.64) (end 71 70.64) (width 1) (layer "B.Cu") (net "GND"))
 (segment (start 105 60.64) (end 111 60.64) (width 1) (layer "B.Cu") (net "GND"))
 (segment (start 109.62 55.64) (end 114 55.64) (width 1) (layer "B.Cu") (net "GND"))
 (segment (start 104 70.34) (end 104 61.64) (width 1) (layer "B.Cu") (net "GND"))
 (segment (start 65.25 71.39) (end 65.25 79.89) (width 1) (layer "B.Cu") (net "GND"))
 (segment (start 66 80.64) (end 75.75 80.64) (width 1) (layer "B.Cu") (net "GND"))
 (segment (start 71 70.64) (end 72.65 68.99) (width 1) (layer "B.Cu") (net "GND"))
 (segment (start 123 58.64) (end 123 76.64) (width 1) (layer "B.Cu") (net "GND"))
 (segment (start 120 55.64) (end 123 58.64) (width 1) (layer "B.Cu") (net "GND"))
 (segment (start 76 80.89) (end 89 80.89) (width 1) (layer "B.Cu") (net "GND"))
 (segment (start 72.65 68.99) (end 72.65 66.64) (width 1) (layer "B.Cu") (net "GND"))
 (segment (start 65.25 79.89) (end 66 80.64) (width 1) (layer "B.Cu") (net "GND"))
 (segment (start 74.95 56.69) (end 67 64.64) (width 1) (layer "B.Cu") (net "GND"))
 (segment (start 109.62 55.64) (end 109.34 55.92) (width 1) (layer "B.Cu") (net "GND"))
 (segment (start 118.75 80.89) (end 102.75 80.89) (width 1) (layer "B.Cu") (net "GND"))
 (segment (start 67 67.64) (end 68 68.64) (width 1) (layer "B.Cu") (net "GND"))
 (segment (start 75.75 80.64) (end 76 80.89) (width 1) (layer "B.Cu") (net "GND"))
 (segment (start 70 78.64) (end 73.46 78.64) (width 1) (layer "B.Cu") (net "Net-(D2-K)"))
 (segment (start 94.38 55.64) (end 79.38 70.64) (width 1) (layer "B.Cu") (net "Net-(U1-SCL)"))
 (segment (start 75.19 69.83) (end 75.19 66.64) (width 1) (layer "B.Cu") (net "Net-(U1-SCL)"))
 (segment (start 76 70.64) (end 75.19 69.83) (width 1) (layer "B.Cu") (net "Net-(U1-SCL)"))
 (segment (start 75.19 63.45) (end 75.19 66.64) (width 1) (layer "B.Cu") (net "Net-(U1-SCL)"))
 (segment (start 80.03 49.68) (end 80.03 58.61) (width 1) (layer "B.Cu") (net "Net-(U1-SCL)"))
 (segment (start 80.03 58.61) (end 75.19 63.45) (width 1) (layer "B.Cu") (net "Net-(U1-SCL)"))
 (segment (start 79.38 70.64) (end 76 70.64) (width 1) (layer "B.Cu") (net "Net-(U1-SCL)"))
 (segment (start 94.38 53.1) (end 87.41 60.07) (width 1) (layer "B.Cu") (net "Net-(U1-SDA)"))
 (segment (start 78 64.64) (end 78 66.37) (width 1) (layer "B.Cu") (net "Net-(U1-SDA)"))
 (segment (start 82.57 49.68) (end 82.57 60.07) (width 1) (layer "B.Cu") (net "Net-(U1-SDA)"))
 (segment (start 87.41 60.07) (end 82.57 60.07) (width 1) (layer "B.Cu") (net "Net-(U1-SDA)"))
 (segment (start 78 66.37) (end 77.73 66.64) (width 1) (layer "B.Cu") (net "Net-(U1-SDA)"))
 (segment (start 82.57 60.07) (end 78 64.64) (width 1) (layer "B.Cu") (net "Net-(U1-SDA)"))
 (segment (start 104 72.64) (end 101 72.64) (width 1) (layer "B.Cu") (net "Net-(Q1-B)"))
 (segment (start 105.27 70.34) (end 105.27 71.37) (width 1) (layer "B.Cu") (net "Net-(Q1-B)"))
 (segment (start 105.27 71.37) (end 104 72.64) (width 1) (layer "B.Cu") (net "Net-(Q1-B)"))
 (segment (start 100.54 72.18) (end 100.54 70.34) (width 1) (layer "B.Cu") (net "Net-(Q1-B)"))
 (segment (start 101 72.64) (end 100.54 72.18) (width 1) (layer "B.Cu") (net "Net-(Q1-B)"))
 (segment (start 93 76.39) (end 95.25 78.64) (width 1) (layer "B.Cu") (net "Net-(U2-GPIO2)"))
 (segment (start 95.25 78.64) (end 113 78.64) (width 1) (layer "B.Cu") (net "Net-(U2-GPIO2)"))
 (segment (start 113.84 65.8) (end 115 66.96) (width 1) (layer "B.Cu") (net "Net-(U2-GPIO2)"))
 (segment (start 113 78.64) (end 115 76.64) (width 1) (layer "B.Cu") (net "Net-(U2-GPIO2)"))
 (segment (start 115 66.96) (end 115 76.64) (width 1) (layer "B.Cu") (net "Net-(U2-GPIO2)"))
 (segment (start 113.84 65.8) (end 109.62 65.8) (width 1) (layer "B.Cu") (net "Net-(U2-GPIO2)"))
 (segment (start 109.62 72.38) (end 109.62 68.34) (width 1) (layer "B.Cu") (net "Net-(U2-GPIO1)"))
 (segment (start 105.61 76.39) (end 109.62 72.38) (width 1) (layer "B.Cu") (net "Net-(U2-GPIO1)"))
 (segment (start 102.75 76.39) (end 105.61 76.39) (width 1) (layer "B.Cu") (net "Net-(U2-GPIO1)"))
 (segment (start 67.46 78.64) (end 73.46 72.64) (width 1) (layer "B.Cu") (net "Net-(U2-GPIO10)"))
 (segment (start 81 72.64) (end 87.84 65.8) (width 1) (layer "B.Cu") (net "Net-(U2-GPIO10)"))
 (segment (start 87.84 65.8) (end 94.38 65.8) (width 1) (layer "B.Cu") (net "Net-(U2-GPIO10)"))
 (segment (start 73.46 72.64) (end 81 72.64) (width 1) (layer "B.Cu") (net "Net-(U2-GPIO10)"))
 (segment (start 80.46 78.64) (end 80.46 77.225787) (width 1) (layer "B.Cu") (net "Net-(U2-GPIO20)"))
 (segment (start 80.46 77.225787) (end 89.345787 68.34) (width 1) (layer "B.Cu") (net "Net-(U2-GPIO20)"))
 (segment (start 89.345787 68.34) (end 94.38 68.34) (width 1) (layer "B.Cu") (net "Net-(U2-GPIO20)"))
 (segment (start 98 70.34) (end 94.92 70.34) (width 1) (layer "B.Cu") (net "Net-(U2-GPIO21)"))
 (segment (start 94.92 70.34) (end 94.38 70.88) (width 1) (layer "B.Cu") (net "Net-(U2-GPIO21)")))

